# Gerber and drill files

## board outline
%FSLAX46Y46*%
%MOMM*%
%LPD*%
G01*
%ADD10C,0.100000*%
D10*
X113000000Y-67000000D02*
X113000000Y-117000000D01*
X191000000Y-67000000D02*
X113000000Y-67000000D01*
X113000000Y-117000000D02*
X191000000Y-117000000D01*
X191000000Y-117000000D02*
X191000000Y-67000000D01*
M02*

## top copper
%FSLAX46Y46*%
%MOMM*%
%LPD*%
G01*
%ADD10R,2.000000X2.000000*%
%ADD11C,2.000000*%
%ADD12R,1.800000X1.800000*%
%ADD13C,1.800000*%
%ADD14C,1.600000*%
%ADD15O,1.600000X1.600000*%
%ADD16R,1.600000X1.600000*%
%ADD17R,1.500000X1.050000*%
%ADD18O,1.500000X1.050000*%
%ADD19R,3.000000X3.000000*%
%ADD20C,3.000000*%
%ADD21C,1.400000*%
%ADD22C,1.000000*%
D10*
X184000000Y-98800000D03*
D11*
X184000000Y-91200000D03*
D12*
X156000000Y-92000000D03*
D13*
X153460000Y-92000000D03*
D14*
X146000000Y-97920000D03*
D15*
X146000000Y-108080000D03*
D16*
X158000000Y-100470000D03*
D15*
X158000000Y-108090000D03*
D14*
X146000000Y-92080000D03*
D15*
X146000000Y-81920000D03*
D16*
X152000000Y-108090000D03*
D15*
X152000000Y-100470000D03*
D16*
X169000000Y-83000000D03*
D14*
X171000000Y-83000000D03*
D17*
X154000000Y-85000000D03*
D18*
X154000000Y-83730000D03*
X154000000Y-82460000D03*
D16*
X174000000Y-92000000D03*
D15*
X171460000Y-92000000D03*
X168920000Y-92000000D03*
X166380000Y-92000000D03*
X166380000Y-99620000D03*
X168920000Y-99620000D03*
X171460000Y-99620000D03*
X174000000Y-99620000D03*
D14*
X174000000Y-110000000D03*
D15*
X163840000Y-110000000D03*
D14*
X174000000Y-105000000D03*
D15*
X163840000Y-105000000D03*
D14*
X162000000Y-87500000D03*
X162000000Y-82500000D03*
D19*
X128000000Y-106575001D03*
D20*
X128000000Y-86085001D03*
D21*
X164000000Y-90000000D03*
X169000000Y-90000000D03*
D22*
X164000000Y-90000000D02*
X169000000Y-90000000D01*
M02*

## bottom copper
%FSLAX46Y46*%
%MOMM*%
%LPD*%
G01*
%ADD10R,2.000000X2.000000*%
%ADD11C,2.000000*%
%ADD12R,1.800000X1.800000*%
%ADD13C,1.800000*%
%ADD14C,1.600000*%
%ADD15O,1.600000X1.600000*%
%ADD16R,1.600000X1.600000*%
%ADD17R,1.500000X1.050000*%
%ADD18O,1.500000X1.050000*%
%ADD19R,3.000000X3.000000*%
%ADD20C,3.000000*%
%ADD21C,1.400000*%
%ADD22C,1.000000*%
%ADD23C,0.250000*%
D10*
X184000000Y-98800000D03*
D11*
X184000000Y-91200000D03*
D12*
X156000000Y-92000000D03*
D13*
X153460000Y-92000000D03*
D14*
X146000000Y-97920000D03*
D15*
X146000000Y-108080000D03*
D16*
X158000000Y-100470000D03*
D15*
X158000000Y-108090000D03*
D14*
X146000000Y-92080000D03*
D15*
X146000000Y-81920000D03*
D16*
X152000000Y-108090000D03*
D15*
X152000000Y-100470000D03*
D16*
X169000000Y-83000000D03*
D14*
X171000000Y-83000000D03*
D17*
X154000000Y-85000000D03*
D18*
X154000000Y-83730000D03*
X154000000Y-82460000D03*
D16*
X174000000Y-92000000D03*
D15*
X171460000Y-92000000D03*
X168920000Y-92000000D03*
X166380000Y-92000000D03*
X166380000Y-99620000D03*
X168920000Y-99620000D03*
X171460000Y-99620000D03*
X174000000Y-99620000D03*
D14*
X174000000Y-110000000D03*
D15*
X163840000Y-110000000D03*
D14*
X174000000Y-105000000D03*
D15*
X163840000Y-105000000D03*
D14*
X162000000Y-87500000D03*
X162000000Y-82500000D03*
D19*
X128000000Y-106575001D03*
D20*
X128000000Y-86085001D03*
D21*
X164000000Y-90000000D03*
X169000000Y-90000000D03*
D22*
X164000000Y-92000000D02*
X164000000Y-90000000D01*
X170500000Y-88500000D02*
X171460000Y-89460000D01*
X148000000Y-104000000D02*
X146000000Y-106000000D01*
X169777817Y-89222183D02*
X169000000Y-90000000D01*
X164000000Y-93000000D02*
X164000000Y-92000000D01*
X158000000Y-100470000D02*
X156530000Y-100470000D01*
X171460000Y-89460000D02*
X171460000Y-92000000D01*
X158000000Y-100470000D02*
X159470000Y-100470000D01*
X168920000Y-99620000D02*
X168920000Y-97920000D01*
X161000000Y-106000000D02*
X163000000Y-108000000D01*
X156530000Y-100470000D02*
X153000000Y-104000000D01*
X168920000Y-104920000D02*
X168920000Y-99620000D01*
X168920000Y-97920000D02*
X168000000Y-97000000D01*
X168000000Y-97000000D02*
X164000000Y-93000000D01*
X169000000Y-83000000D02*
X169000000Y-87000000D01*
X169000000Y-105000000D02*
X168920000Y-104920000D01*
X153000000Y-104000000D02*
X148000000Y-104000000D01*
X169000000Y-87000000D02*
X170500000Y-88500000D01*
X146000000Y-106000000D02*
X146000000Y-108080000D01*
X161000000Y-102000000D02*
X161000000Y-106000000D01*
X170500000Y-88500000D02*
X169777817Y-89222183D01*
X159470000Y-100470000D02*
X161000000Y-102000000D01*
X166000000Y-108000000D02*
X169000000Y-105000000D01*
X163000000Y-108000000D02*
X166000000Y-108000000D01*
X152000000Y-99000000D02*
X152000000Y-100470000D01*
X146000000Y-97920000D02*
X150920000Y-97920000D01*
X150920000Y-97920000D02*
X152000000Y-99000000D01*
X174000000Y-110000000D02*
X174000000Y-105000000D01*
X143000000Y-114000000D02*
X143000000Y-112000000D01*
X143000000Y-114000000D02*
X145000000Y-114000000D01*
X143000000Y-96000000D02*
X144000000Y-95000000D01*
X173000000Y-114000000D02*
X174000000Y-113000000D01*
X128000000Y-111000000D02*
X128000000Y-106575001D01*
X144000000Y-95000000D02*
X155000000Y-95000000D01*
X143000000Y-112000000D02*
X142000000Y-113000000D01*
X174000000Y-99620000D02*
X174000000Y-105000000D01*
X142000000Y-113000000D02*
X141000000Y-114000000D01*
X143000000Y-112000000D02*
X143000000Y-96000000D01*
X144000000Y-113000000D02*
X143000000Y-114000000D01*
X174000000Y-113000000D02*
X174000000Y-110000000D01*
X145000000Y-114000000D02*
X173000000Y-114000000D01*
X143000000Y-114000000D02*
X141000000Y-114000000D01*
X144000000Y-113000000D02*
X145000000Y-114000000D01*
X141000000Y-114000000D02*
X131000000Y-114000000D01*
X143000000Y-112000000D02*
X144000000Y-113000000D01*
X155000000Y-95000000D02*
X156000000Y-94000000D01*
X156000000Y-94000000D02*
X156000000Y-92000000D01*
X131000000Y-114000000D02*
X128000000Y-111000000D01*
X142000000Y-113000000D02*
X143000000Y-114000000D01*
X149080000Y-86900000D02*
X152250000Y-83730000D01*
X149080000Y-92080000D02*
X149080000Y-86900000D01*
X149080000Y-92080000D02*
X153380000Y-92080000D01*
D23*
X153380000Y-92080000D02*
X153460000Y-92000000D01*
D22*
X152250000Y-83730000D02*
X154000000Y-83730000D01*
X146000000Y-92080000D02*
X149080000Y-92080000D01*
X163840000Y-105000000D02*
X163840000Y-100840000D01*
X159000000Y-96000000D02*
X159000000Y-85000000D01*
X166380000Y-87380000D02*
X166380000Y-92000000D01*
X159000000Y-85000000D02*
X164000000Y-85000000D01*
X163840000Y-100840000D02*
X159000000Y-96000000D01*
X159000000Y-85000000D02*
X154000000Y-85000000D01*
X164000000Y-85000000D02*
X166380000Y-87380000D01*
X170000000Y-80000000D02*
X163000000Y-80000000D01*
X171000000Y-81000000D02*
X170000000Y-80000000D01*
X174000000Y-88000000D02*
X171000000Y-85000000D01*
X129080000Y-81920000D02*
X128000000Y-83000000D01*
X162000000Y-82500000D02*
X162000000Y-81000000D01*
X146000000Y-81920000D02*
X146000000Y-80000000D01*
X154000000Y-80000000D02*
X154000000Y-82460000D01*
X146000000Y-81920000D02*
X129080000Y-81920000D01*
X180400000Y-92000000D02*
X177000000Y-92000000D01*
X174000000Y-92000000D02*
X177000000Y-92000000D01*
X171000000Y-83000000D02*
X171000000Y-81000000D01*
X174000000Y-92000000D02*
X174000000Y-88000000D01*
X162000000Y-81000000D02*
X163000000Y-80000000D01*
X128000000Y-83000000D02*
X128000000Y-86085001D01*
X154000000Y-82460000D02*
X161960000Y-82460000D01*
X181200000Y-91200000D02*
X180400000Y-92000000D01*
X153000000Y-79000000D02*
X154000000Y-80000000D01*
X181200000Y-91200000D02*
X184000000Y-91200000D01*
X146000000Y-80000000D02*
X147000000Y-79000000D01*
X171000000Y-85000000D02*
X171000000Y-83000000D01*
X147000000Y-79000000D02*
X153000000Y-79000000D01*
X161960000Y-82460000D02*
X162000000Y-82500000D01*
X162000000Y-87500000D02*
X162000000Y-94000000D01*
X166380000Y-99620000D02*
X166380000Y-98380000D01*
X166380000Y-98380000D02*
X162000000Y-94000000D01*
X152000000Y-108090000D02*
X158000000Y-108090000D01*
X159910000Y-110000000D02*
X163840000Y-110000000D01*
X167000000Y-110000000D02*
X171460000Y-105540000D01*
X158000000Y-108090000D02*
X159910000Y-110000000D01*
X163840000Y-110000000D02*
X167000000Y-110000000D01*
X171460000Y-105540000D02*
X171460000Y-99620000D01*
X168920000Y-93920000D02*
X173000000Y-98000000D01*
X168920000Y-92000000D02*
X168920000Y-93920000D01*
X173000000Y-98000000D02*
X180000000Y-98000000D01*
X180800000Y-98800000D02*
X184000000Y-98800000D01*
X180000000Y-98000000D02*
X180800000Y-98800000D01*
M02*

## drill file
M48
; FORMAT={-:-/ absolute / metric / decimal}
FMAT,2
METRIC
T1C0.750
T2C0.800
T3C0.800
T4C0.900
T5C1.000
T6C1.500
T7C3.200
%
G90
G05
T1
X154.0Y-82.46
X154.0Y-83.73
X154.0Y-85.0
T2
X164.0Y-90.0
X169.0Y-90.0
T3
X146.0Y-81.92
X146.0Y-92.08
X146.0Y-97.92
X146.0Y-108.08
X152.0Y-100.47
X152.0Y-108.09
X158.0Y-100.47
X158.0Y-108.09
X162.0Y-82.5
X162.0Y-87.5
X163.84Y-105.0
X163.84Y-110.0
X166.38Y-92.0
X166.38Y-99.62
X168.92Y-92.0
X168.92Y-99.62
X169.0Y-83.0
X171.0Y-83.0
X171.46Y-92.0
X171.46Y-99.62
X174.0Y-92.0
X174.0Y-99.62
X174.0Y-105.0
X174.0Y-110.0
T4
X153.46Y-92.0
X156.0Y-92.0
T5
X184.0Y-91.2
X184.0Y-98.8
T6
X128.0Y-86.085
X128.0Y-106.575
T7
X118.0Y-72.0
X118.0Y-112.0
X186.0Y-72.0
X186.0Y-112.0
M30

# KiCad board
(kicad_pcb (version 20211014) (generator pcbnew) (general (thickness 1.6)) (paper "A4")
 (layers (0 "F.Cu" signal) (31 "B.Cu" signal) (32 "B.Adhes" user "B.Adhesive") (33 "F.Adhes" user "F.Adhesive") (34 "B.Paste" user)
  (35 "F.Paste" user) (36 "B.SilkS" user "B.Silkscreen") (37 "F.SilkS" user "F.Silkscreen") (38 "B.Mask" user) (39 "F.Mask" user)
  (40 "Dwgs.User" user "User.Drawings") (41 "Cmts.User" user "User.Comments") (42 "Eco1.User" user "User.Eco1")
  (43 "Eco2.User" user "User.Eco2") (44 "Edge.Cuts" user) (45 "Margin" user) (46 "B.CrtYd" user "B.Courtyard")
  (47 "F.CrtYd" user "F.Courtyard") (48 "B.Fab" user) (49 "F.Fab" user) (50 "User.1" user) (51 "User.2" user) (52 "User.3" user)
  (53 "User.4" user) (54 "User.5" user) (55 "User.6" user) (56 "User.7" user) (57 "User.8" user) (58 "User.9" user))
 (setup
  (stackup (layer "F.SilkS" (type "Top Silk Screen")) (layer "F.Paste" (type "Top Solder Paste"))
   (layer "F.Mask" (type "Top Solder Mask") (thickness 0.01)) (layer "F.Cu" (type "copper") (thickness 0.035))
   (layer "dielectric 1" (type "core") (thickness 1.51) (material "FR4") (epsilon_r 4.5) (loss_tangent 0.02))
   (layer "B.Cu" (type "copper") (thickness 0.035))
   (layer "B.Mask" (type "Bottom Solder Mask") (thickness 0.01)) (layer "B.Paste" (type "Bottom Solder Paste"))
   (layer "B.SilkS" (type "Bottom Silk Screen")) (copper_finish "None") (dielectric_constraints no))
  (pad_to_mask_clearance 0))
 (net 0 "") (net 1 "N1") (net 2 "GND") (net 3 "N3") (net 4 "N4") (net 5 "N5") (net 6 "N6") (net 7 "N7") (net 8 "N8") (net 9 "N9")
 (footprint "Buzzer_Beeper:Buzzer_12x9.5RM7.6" (layer "F.Cu") (at 184 98.8 90)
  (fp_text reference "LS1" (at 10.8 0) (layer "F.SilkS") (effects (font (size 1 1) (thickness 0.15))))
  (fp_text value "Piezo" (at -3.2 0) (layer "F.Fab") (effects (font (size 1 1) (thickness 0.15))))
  (pad "1" thru_hole rect (at 0 0 90) (size 2 2) (drill 1) (layers *.Cu *.Mask) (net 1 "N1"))
  (pad "2" thru_hole circle (at 7.6 0 90) (size 2 2) (drill 1) (layers *.Cu *.Mask) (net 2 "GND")))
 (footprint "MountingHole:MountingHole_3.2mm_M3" (layer "F.Cu") (at 118 72)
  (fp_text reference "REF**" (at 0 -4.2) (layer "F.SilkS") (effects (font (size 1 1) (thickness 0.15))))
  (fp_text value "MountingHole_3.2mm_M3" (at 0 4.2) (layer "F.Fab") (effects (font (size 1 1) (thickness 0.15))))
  (pad "" np_thru_hole circle (at 0 0) (size 3.2 3.2) (drill 3.2) (layers *.Cu *.Mask)))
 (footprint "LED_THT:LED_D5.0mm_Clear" (layer "F.Cu") (at 156 92 180)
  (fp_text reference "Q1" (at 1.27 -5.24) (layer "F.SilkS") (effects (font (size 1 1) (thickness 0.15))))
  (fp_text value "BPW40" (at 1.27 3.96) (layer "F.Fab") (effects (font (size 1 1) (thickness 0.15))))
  (pad "1" thru_hole rect (at 0 0 180) (size 1.8 1.8) (drill 0.9) (layers *.Cu *.Mask) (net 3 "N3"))
  (pad "2" thru_hole circle (at 2.54 0 180) (size 1.8 1.8) (drill 0.9) (layers *.Cu *.Mask) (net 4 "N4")))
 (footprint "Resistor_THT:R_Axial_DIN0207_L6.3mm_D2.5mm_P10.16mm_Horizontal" (layer "F.Cu") (at 146 97.92 -90)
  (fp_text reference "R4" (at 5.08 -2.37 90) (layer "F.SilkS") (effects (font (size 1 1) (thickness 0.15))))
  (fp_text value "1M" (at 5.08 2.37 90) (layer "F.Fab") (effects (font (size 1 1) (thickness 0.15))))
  (pad "1" thru_hole circle (at 0 0 270) (size 1.6 1.6) (drill 0.8) (layers *.Cu *.Mask) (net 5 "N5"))
  (pad "2" thru_hole oval (at 10.16 0 270) (size 1.6 1.6) (drill 0.8) (layers *.Cu *.Mask) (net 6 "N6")))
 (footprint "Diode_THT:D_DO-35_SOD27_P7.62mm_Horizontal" (layer "F.Cu") (at 158 100.47 -90)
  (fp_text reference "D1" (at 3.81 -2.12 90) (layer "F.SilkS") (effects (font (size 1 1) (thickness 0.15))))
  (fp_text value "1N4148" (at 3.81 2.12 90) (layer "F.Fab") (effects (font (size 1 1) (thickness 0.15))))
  (pad "1" thru_hole rect (at 0 0 270) (size 1.6 1.6) (drill 0.8) (layers *.Cu *.Mask) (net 6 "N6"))
  (pad "2" thru_hole oval (at 7.62 0 270) (size 1.6 1.6) (drill 0.8) (layers *.Cu *.Mask) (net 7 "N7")))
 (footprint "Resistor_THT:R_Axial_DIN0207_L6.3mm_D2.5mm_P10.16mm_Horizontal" (layer "F.Cu") (at 146 92.08 90)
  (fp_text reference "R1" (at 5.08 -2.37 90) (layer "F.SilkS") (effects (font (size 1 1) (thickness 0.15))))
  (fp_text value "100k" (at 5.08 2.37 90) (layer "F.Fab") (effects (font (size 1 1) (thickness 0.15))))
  (pad "1" thru_hole circle (at 0 0 90) (size 1.6 1.6) (drill 0.8) (layers *.Cu *.Mask) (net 4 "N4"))
  (pad "2" thru_hole oval (at 10.16 0 90) (size 1.6 1.6) (drill 0.8) (layers *.Cu *.Mask) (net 2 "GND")))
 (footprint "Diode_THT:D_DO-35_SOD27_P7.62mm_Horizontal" (layer "F.Cu") (at 152 108.09 90)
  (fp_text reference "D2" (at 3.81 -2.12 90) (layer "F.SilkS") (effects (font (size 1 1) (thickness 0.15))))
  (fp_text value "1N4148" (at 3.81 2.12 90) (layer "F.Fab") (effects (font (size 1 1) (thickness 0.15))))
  (pad "1" thru_hole rect (at 0 0 90) (size 1.6 1.6) (drill 0.8) (layers *.Cu *.Mask) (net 7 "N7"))
  (pad "2" thru_hole oval (at 7.62 0 90) (size 1.6 1.6) (drill 0.8) (layers *.Cu *.Mask) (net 5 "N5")))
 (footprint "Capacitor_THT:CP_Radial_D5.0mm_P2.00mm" (layer "F.Cu") (at 169 83)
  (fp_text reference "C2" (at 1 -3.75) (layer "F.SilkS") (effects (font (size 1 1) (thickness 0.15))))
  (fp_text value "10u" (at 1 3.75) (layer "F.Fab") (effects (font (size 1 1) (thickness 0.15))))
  (pad "1" thru_hole rect (at 0 0) (size 1.6 1.6) (drill 0.8) (layers *.Cu *.Mask) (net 6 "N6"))
  (pad "2" thru_hole circle (at 2 0) (size 1.6 1.6) (drill 0.8) (layers *.Cu *.Mask) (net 2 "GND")))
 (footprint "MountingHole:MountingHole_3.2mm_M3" (layer "F.Cu") (at 118 112)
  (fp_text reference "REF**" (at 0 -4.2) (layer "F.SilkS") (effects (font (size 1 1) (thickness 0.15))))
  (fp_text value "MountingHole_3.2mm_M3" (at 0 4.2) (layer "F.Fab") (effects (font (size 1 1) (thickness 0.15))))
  (pad "" np_thru_hole circle (at 0 0) (size 3.2 3.2) (drill 3.2) (layers F&B.Cu *.Mask)))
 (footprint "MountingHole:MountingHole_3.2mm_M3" (layer "F.Cu") (at 186 112)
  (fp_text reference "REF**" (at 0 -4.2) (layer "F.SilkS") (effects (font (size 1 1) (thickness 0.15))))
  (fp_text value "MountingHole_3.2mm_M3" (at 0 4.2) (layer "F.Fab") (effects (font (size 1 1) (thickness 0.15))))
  (pad "" np_thru_hole circle (at 0 0) (size 3.2 3.2) (drill 3.2) (layers F&B.Cu *.Mask)))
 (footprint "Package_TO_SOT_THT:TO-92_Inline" (layer "F.Cu") (at 154 85 90)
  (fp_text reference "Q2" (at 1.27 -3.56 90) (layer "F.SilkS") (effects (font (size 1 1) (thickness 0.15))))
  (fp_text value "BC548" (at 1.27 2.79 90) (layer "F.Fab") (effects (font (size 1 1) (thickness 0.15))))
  (pad "1" thru_hole rect (at 0 0 90) (size 1.05 1.5) (drill 0.75) (layers *.Cu *.Mask) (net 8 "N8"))
  (pad "2" thru_hole oval (at 1.27 0 90) (size 1.05 1.5) (drill 0.75) (layers *.Cu *.Mask) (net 4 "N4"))
  (pad "3" thru_hole oval (at 2.54 0 90) (size 1.05 1.5) (drill 0.75) (layers *.Cu *.Mask) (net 2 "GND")))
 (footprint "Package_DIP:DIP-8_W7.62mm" (layer "F.Cu") (at 174 92 -90)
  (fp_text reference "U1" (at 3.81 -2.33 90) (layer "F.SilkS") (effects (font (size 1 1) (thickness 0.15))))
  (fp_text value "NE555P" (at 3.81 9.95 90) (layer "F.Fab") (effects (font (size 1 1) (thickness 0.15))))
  (pad "1" thru_hole rect (at 0 0 270) (size 1.6 1.6) (drill 0.8) (layers *.Cu *.Mask) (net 2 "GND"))
  (pad "2" thru_hole oval (at 0 2.54 270) (size 1.6 1.6) (drill 0.8) (layers *.Cu *.Mask) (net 6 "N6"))
  (pad "3" thru_hole oval (at 0 5.08 270) (size 1.6 1.6) (drill 0.8) (layers *.Cu *.Mask) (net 1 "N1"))
  (pad "4" thru_hole oval (at 0 7.62 270) (size 1.6 1.6) (drill 0.8) (layers *.Cu *.Mask) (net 8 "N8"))
  (pad "5" thru_hole oval (at 7.62 7.62 270) (size 1.6 1.6) (drill 0.8) (layers *.Cu *.Mask) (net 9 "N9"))
  (pad "6" thru_hole oval (at 7.62 5.08 270) (size 1.6 1.6) (drill 0.8) (layers *.Cu *.Mask) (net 6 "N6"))
  (pad "7" thru_hole oval (at 7.62 2.54 270) (size 1.6 1.6) (drill 0.8) (layers *.Cu *.Mask) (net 7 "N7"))
  (pad "8" thru_hole oval (at 7.62 0 270) (size 1.6 1.6) (drill 0.8) (layers *.Cu *.Mask) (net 3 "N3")))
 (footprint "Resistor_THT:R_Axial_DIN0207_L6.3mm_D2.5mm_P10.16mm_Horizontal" (layer "F.Cu") (at 174 110 180)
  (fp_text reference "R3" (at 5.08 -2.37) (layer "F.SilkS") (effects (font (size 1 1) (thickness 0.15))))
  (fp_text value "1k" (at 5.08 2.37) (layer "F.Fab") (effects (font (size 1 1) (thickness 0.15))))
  (pad "1" thru_hole circle (at 0 0 180) (size 1.6 1.6) (drill 0.8) (layers *.Cu *.Mask) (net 3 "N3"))
  (pad "2" thru_hole oval (at 10.16 0 180) (size 1.6 1.6) (drill 0.8) (layers *.Cu *.Mask) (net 7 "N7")))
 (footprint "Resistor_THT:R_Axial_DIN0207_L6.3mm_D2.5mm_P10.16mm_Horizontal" (layer "F.Cu") (at 174 105 180)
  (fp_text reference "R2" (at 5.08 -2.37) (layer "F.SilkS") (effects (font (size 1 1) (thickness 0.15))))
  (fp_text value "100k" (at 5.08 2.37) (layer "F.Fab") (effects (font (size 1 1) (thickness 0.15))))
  (pad "1" thru_hole circle (at 0 0 180) (size 1.6 1.6) (drill 0.8) (layers *.Cu *.Mask) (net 3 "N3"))
  (pad "2" thru_hole oval (at 10.16 0 180) (size 1.6 1.6) (drill 0.8) (layers *.Cu *.Mask) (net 8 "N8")))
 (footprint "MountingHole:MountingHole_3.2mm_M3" (layer "F.Cu") (at 186 72)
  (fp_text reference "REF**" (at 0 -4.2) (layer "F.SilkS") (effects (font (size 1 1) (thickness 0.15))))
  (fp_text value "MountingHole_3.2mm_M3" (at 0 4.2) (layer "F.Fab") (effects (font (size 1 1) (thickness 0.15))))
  (pad "" np_thru_hole circle (at 0 0) (size 3.2 3.2) (drill 3.2) (layers F&B.Cu *.Mask)))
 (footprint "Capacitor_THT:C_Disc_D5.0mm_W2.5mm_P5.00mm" (layer "F.Cu") (at 162 87.5 90)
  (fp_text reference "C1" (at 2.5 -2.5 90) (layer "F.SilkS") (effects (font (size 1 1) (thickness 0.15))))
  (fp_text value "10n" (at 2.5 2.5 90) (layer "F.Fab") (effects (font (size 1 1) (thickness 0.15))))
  (pad "1" thru_hole circle (at 0 0 90) (size 1.6 1.6) (drill 0.8) (layers *.Cu *.Mask) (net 9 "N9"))
  (pad "2" thru_hole circle (at 5 0 90) (size 1.6 1.6) (drill 0.8) (layers *.Cu *.Mask) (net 2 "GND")))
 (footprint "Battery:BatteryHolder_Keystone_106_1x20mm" (layer "B.Cu") (at 128 106.575001 90)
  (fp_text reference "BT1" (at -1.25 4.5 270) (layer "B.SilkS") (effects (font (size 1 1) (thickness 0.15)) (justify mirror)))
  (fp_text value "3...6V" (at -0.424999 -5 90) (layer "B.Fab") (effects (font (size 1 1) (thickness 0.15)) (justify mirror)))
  (pad "1" thru_hole rect (at 0 0 90) (size 3 3) (drill 1.5) (layers *.Cu *.Mask) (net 3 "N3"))
  (pad "2" thru_hole circle (at 20.49 0 90) (size 3 3) (drill 1.5) (layers *.Cu *.Mask) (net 2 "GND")))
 (gr_line (start 113 67) (end 113 117) (layer "Edge.Cuts") (width 0.1))
 (gr_line (start 191 67) (end 113 67) (layer "Edge.Cuts") (width 0.1))
 (gr_line (start 113 117) (end 191 117) (layer "Edge.Cuts") (width 0.1))
 (gr_line (start 191 117) (end 191 67) (layer "Edge.Cuts") (width 0.1))
 (segment (start 164 90) (end 169 90) (width 1) (layer "F.Cu") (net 6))
 (via (at 164 90) (size 1.4) (drill 0.8) (layers "F.Cu" "B.Cu") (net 6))
 (via (at 169 90) (size 1.4) (drill 0.8) (layers "F.Cu" "B.Cu") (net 6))
 (segment (start 164 92) (end 164 90) (width 1) (layer "B.Cu") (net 6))
 (segment (start 170.5 88.5) (end 171.46 89.46) (width 1) (layer "B.Cu") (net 6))
 (segment (start 148 104) (end 146 106) (width 1) (layer "B.Cu") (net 6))
 (segment (start 169.777817 89.222183) (end 169 90) (width 1) (layer "B.Cu") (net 6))
 (segment (start 164 93) (end 164 92) (width 1) (layer "B.Cu") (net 6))
 (segment (start 158 100.47) (end 156.53 100.47) (width 1) (layer "B.Cu") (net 6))
 (segment (start 171.46 89.46) (end 171.46 92) (width 1) (layer "B.Cu") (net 6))
 (segment (start 158 100.47) (end 159.47 100.47) (width 1) (layer "B.Cu") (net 6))
 (segment (start 168.92 99.62) (end 168.92 97.92) (width 1) (layer "B.Cu") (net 6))
 (segment (start 161 106) (end 163 108) (width 1) (layer "B.Cu") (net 6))
 (segment (start 156.53 100.47) (end 153 104) (width 1) (layer "B.Cu") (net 6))
 (segment (start 168.92 104.92) (end 168.92 99.62) (width 1) (layer "B.Cu") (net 6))
 (segment (start 168.92 97.92) (end 168 97) (width 1) (layer "B.Cu") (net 6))
 (segment (start 168 97) (end 164 93) (width 1) (layer "B.Cu") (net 6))
 (segment (start 169 83) (end 169 87) (width 1) (layer "B.Cu") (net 6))
 (segment (start 169 105) (end 168.92 104.92) (width 1) (layer "B.Cu") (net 6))
 (segment (start 153 104) (end 148 104) (width 1) (layer "B.Cu") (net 6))
 (segment (start 169 87) (end 170.5 88.5) (width 1) (layer "B.Cu") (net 6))
 (segment (start 146 106) (end 146 108.08) (width 1) (layer "B.Cu") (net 6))
 (segment (start 161 102) (end 161 106) (width 1) (layer "B.Cu") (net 6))
 (segment (start 170.5 88.5) (end 169.777817 89.222183) (width 1) (layer "B.Cu") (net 6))
 (segment (start 159.47 100.47) (end 161 102) (width 1) (layer "B.Cu") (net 6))
 (segment (start 166 108) (end 169 105) (width 1) (layer "B.Cu") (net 6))
 (segment (start 163 108) (end 166 108) (width 1) (layer "B.Cu") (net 6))
 (segment (start 152 99) (end 152 100.47) (width 1) (layer "B.Cu") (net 5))
 (segment (start 146 97.92) (end 150.92 97.92) (width 1) (layer "B.Cu") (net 5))
 (segment (start 150.92 97.92) (end 152 99) (width 1) (layer "B.Cu") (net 5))
 (segment (start 174 110) (end 174 105) (width 1) (layer "B.Cu") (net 3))
 (segment (start 143 114) (end 143 112) (width 1) (layer "B.Cu") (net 3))
 (segment (start 143 114) (end 145 114) (width 1) (layer "B.Cu") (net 3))
 (segment (start 143 96) (end 144 95) (width 1) (layer "B.Cu") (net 3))
 (segment (start 173 114) (end 174 113) (width 1) (layer "B.Cu") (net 3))
 (segment (start 128 111) (end 128 106.575001) (width 1) (layer "B.Cu") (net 3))
 (segment (start 144 95) (end 155 95) (width 1) (layer "B.Cu") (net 3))
 (segment (start 143 112) (end 142 113) (width 1) (layer "B.Cu") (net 3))
 (segment (start 174 99.62) (end 174 105) (width 1) (layer "B.Cu") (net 3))
 (segment (start 142 113) (end 141 114) (width 1) (layer "B.Cu") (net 3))
 (segment (start 143 112) (end 143 96) (width 1) (layer "B.Cu") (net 3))
 (segment (start 144 113) (end 143 114) (width 1) (layer "B.Cu") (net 3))
 (segment (start 174 113) (end 174 110) (width 1) (layer "B.Cu") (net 3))
 (segment (start 145 114) (end 173 114) (width 1) (layer "B.Cu") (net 3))
 (segment (start 143 114) (end 141 114) (width 1) (layer "B.Cu") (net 3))
 (segment (start 144 113) (end 145 114) (width 1) (layer "B.Cu") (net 3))
 (segment (start 141 114) (end 131 114) (width 1) (layer "B.Cu") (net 3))
 (segment (start 143 112) (end 144 113) (width 1) (layer "B.Cu") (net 3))
 (segment (start 155 95) (end 156 94) (width 1) (layer "B.Cu") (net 3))
 (segment (start 156 94) (end 156 92) (width 1) (layer "B.Cu") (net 3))
 (segment (start 131 114) (end 128 111) (width 1) (layer "B.Cu") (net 3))
 (segment (start 142 113) (end 143 114) (width 1) (layer "B.Cu") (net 3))
 (segment (start 149.08 86.9) (end 152.25 83.73) (width 1) (layer "B.Cu") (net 4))
 (segment (start 149.08 92.08) (end 149.08 86.9) (width 1) (layer "B.Cu") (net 4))
 (segment (start 149.08 92.08) (end 153.38 92.08) (width 1) (layer "B.Cu") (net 4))
 (segment (start 153.38 92.08) (end 153.46 92) (width 0.25) (layer "B.Cu") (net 4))
 (segment (start 152.25 83.73) (end 154 83.73) (width 1) (layer "B.Cu") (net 4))
 (segment (start 146 92.08) (end 149.08 92.08) (width 1) (layer "B.Cu") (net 4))
 (segment (start 163.84 105) (end 163.84 100.84) (width 1) (layer "B.Cu") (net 8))
 (segment (start 159 96) (end 159 85) (width 1) (layer "B.Cu") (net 8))
 (segment (start 166.38 87.38) (end 166.38 92) (width 1) (layer "B.Cu") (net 8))
 (segment (start 159 85) (end 164 85) (width 1) (layer "B.Cu") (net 8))
 (segment (start 163.84 100.84) (end 159 96) (width 1) (layer "B.Cu") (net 8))
 (segment (start 159 85) (end 154 85) (width 1) (layer "B.Cu") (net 8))
 (segment (start 164 85) (end 166.38 87.38) (width 1) (layer "B.Cu") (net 8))
 (segment (start 170 80) (end 163 80) (width 1) (layer "B.Cu") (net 2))
 (segment (start 171 81) (end 170 80) (width 1) (layer "B.Cu") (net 2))
 (segment (start 174 88) (end 171 85) (width 1) (layer "B.Cu") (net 2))
 (segment (start 129.08 81.92) (end 128 83) (width 1) (layer "B.Cu") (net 2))
 (segment (start 162 82.5) (end 162 81) (width 1) (layer "B.Cu") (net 2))
 (segment (start 146 81.92) (end 146 80) (width 1) (layer "B.Cu") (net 2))
 (segment (start 154 80) (end 154 82.46) (width 1) (layer "B.Cu") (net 2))
 (segment (start 146 81.92) (end 129.08 81.92) (width 1) (layer "B.Cu") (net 2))
 (segment (start 180.4 92) (end 177 92) (width 1) (layer "B.Cu") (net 2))
 (segment (start 174 92) (end 177 92) (width 1) (layer "B.Cu") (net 2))
 (segment (start 171 83) (end 171 81) (width 1) (layer "B.Cu") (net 2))
 (segment (start 174 92) (end 174 88) (width 1) (layer "B.Cu") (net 2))
 (segment (start 162 81) (end 163 80) (width 1) (layer "B.Cu") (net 2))
 (segment (start 128 83) (end 128 86.085001) (width 1) (layer "B.Cu") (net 2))
 (segment (start 154 82.46) (end 161.96 82.46) (width 1) (layer "B.Cu") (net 2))
 (segment (start 181.2 91.2) (end 180.4 92) (width 1) (layer "B.Cu") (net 2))
 (segment (start 153 79) (end 154 80) (width 1) (layer "B.Cu") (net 2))
 (segment (start 181.2 91.2) (end 184 91.2) (width 1) (layer "B.Cu") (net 2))
 (segment (start 146 80) (end 147 79) (width 1) (layer "B.Cu") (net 2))
 (segment (start 171 85) (end 171 83) (width 1) (layer "B.Cu") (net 2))
 (segment (start 147 79) (end 153 79) (width 1) (layer "B.Cu") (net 2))
 (segment (start 161.96 82.46) (end 162 82.5) (width 1) (layer "B.Cu") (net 2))
 (segment (start 162 87.5) (end 162 94) (width 1) (layer "B.Cu") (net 9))
 (segment (start 166.38 99.62) (end 166.38 98.38) (width 1) (layer "B.Cu") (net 9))
 (segment (start 166.38 98.38) (end 162 94) (width 1) (layer "B.Cu") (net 9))
 (segment (start 152 108.09) (end 158 108.09) (width 1) (layer "B.Cu") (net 7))
 (segment (start 159.91 110) (end 163.84 110) (width 1) (layer "B.Cu") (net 7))
 (segment (start 167 110) (end 171.46 105.54) (width 1) (layer "B.Cu") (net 7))
 (segment (start 158 108.09) (end 159.91 110) (width 1) (layer "B.Cu") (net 7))
 (segment (start 163.84 110) (end 167 110) (width 1) (layer "B.Cu") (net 7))
 (segment (start 171.46 105.54) (end 171.46 99.62) (width 1) (layer "B.Cu") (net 7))
 (segment (start 168.92 93.92) (end 173 98) (width 1) (layer "B.Cu") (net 1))
 (segment (start 168.92 92) (end 168.92 93.92) (width 1) (layer "B.Cu") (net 1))
 (segment (start 173 98) (end 180 98) (width 1) (layer "B.Cu") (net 1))
 (segment (start 180.8 98.8) (end 184 98.8) (width 1) (layer "B.Cu") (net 1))
 (segment (start 180 98) (end 180.8 98.8) (width 1) (layer "B.Cu") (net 1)))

